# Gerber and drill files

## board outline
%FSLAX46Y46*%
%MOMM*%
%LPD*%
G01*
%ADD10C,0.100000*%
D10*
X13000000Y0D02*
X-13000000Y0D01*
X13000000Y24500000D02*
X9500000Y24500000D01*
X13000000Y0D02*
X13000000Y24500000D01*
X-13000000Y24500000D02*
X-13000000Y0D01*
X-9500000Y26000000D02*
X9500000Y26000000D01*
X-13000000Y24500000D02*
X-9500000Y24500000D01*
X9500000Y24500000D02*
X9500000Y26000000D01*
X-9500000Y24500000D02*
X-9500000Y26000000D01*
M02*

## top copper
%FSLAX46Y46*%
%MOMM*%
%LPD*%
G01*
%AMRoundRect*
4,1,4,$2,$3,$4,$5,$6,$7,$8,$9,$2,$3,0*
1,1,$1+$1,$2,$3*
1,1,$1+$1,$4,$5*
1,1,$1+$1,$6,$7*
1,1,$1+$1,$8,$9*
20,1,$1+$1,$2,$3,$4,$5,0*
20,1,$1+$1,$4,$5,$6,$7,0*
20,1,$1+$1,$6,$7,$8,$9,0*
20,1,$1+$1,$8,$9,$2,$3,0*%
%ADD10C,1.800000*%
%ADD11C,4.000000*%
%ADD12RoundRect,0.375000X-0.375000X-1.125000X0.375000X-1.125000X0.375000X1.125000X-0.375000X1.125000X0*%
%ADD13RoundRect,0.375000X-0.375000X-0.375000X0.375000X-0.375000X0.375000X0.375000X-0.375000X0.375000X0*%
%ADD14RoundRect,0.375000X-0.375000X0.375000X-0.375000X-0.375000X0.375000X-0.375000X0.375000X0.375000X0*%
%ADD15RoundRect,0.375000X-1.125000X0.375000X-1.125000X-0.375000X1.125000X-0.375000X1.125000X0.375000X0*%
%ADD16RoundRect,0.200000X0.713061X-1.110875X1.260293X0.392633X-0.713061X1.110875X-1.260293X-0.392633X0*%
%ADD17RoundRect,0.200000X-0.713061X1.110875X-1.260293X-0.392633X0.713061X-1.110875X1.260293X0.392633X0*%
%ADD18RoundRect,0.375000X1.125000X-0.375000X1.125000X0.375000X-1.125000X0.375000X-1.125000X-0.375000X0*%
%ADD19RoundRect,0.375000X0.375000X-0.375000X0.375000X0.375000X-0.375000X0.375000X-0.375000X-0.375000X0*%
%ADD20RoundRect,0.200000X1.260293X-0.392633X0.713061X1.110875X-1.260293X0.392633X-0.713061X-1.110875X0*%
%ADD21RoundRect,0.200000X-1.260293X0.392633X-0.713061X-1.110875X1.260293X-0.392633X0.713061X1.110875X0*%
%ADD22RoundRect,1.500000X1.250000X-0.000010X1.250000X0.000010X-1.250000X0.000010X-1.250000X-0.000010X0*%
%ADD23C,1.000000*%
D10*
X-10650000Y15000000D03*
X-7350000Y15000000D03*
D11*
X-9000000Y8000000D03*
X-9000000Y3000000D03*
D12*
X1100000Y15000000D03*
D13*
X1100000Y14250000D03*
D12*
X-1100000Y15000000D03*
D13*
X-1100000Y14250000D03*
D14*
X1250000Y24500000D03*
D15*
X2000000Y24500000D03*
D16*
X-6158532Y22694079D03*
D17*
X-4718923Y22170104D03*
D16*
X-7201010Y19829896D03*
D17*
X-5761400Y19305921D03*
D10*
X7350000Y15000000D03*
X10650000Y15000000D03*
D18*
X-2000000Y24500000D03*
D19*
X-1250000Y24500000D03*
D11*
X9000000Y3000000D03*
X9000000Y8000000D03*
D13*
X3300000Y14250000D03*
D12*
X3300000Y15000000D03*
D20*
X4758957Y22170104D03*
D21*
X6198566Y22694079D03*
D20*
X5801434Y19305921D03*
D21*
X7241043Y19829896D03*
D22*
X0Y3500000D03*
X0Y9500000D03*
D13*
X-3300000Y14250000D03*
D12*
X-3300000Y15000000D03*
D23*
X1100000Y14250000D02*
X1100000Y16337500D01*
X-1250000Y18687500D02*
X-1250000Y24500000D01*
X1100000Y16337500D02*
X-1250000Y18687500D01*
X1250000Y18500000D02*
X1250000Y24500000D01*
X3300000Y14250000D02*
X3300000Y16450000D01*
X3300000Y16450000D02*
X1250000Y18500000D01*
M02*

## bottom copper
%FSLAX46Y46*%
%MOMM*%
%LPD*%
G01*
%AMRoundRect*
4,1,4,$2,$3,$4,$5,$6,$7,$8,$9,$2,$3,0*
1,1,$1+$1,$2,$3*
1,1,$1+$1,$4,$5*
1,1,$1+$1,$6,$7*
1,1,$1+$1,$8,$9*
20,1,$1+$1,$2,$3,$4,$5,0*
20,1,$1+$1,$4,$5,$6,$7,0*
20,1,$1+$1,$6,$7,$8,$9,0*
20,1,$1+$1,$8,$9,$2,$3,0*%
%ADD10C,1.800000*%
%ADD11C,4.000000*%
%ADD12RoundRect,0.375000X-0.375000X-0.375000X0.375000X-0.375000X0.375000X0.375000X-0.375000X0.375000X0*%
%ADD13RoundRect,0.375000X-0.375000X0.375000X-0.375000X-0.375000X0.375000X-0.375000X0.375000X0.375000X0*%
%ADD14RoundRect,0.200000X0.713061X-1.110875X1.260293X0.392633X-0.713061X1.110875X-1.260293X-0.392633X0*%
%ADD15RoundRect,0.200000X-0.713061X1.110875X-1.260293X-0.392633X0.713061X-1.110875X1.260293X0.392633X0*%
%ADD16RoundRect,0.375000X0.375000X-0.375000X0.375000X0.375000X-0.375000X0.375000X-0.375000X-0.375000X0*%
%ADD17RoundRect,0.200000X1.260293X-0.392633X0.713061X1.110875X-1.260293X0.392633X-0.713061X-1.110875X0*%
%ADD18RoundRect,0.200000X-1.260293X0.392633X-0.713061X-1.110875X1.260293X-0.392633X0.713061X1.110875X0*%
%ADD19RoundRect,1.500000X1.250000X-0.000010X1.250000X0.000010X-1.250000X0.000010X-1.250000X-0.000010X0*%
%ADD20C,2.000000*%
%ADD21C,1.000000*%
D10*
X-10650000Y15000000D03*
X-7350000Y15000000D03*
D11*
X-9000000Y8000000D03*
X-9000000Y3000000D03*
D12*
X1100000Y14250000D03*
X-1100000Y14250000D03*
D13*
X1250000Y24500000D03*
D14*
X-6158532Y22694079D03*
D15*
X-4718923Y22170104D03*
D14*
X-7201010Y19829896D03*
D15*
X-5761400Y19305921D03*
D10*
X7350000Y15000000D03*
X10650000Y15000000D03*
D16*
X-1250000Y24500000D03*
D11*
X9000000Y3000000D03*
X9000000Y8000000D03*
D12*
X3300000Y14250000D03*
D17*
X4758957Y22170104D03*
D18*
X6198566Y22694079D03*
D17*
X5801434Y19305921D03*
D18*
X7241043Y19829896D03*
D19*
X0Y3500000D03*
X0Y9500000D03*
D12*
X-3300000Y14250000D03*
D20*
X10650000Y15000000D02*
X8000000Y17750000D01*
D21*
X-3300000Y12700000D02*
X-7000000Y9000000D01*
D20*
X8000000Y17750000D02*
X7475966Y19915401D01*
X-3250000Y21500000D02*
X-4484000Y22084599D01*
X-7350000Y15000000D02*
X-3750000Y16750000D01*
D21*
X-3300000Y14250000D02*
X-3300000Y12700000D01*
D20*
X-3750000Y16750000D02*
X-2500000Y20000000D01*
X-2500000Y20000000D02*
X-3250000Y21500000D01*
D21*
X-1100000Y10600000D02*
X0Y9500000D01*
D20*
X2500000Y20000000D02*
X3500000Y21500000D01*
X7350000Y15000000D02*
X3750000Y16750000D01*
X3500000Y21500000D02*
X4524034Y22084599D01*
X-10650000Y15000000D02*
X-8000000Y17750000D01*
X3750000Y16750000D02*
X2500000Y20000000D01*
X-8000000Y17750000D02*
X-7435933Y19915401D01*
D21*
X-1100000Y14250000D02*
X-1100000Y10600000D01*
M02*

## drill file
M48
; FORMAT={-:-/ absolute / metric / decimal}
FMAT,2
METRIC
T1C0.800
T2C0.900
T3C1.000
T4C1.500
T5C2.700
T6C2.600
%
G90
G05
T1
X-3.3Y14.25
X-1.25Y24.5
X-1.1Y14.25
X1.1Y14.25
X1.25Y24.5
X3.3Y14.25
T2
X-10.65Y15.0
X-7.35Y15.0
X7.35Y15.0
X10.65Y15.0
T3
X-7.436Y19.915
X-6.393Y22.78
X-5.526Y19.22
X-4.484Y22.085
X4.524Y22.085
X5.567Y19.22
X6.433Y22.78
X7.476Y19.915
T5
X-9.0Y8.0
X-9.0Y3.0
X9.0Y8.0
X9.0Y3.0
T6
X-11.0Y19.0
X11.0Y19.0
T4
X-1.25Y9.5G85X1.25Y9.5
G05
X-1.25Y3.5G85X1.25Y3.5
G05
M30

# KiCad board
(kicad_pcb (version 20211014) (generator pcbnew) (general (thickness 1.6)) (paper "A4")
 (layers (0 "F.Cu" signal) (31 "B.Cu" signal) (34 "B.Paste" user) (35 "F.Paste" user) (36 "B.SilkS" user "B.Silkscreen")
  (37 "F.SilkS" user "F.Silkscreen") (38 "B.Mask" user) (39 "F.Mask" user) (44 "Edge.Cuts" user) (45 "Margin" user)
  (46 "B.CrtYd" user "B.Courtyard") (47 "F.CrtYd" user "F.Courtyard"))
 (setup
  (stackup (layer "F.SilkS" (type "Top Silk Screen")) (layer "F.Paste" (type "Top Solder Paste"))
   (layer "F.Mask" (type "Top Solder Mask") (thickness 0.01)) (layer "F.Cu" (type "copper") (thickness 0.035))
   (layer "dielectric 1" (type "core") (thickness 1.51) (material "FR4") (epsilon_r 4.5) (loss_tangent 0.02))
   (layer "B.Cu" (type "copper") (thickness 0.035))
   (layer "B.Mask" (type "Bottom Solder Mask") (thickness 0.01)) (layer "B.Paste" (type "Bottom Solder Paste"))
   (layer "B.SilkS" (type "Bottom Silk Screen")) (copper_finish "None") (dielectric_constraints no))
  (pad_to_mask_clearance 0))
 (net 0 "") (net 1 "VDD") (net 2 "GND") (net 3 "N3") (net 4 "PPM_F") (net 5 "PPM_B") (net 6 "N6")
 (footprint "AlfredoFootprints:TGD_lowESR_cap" (layer "F.Cu") (at -9 -15)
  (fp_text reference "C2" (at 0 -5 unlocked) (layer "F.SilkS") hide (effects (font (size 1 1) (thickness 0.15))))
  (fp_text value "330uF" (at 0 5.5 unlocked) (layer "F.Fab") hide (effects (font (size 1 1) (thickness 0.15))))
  (pad "1" thru_hole circle (at -1.65 0) (size 1.8 1.8) (drill 0.9) (layers *.Cu *.Mask) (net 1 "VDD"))
  (pad "2" thru_hole circle (at 1.65 0) (size 1.8 1.8) (drill 0.9) (layers *.Cu *.Mask) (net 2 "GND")))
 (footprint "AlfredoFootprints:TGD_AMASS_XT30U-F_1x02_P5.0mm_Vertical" (layer "F.Cu") (at -9 -5.5 -90)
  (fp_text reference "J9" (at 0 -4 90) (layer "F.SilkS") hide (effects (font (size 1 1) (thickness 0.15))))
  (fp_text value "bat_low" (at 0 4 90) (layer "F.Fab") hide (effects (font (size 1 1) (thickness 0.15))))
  (pad "1" thru_hole circle (at -2.5 0 270) (size 4 4) (drill 2.7) (layers *.Cu *.Mask) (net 2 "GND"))
  (pad "2" thru_hole circle (at 2.5 0 270) (size 4 4) (drill 2.7) (layers *.Cu *.Mask) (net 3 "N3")))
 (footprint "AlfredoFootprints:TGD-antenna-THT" (layer "F.Cu") (at 1.1 -15)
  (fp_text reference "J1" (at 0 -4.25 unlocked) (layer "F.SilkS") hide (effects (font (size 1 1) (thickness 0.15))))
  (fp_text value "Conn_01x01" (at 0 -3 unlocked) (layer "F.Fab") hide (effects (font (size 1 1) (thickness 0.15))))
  (pad "1" smd roundrect (at 0 0) (size 1.5 3) (layers "F.Cu" "F.Paste" "F.Mask") (roundrect_rratio 0.25) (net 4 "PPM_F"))
  (pad "1" thru_hole roundrect (at 0 0.75) (size 1.5 1.5) (drill 0.8) (layers *.Cu *.Mask) (roundrect_rratio 0.25) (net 4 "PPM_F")))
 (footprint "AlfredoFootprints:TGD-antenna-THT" (layer "F.Cu") (at -1.1 -15)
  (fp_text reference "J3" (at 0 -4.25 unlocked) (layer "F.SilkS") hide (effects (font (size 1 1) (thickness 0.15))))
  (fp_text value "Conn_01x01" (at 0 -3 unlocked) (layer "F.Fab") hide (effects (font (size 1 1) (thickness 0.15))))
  (pad "1" smd roundrect (at 0 0) (size 1.5 3) (layers "F.Cu" "F.Paste" "F.Mask") (roundrect_rratio 0.25) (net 1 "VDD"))
  (pad "1" thru_hole roundrect (at 0 0.75) (size 1.5 1.5) (drill 0.8) (layers *.Cu *.Mask) (roundrect_rratio 0.25) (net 1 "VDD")))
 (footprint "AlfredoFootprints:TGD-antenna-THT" (layer "F.Cu") (at 2 -24.5 -90)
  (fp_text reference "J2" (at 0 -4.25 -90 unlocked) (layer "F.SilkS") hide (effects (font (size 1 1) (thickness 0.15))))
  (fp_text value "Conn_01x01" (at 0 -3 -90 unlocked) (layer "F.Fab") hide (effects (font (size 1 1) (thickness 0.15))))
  (pad "1" thru_hole roundrect (at 0 0.75 270) (size 1.5 1.5) (drill 0.8) (layers *.Cu *.Mask) (roundrect_rratio 0.25) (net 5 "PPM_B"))
  (pad "1" smd roundrect (at 0 0 270) (size 1.5 3) (layers "F.Cu" "F.Paste" "F.Mask") (roundrect_rratio 0.25) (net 5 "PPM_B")))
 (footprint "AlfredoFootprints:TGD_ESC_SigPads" (layer "F.Cu") (at -4.484 -22.084599 -110)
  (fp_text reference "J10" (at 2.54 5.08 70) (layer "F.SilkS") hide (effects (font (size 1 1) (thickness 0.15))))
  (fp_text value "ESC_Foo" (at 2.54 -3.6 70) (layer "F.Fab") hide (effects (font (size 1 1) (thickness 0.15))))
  (pad "1" thru_hole roundrect locked (at 0 2.032 70) (size 2 2.5) (drill 1 (offset 0 0.25)) (layers *.Cu *.Mask) (roundrect_rratio 0.1)
   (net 2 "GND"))
  (pad "1" thru_hole roundrect locked (at 0 0 250) (size 2 2.5) (drill 1 (offset 0 0.25)) (layers *.Cu *.Mask) (roundrect_rratio 0.1)
   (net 2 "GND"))
  (pad "2" thru_hole roundrect locked (at 3.048 2.032 70) (size 2 2.5) (drill 1 (offset 0 0.25)) (layers *.Cu *.Mask) (roundrect_rratio 0.1)
   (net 1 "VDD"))
  (pad "2" thru_hole roundrect locked (at 3.048 0 250) (size 2 2.5) (drill 1 (offset 0 0.25)) (layers *.Cu *.Mask) (roundrect_rratio 0.1)
   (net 1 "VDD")))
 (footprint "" (layer "F.Cu") (at 11 -19)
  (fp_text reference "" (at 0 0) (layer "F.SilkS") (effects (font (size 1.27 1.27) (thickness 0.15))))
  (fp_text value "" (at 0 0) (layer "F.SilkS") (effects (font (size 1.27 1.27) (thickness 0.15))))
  (pad "" np_thru_hole circle locked (at 0 0) (size 2.6 2.6) (drill 2.6) (layers F&B.Cu *.Mask)))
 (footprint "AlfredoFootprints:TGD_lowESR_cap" (layer "F.Cu") (at 9 -15)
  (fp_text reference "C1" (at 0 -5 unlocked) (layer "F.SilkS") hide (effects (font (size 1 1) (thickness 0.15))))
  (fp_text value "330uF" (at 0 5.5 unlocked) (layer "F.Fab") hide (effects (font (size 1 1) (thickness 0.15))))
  (pad "1" thru_hole circle (at -1.65 0) (size 1.8 1.8) (drill 0.9) (layers *.Cu *.Mask) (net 1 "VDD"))
  (pad "2" thru_hole circle (at 1.65 0) (size 1.8 1.8) (drill 0.9) (layers *.Cu *.Mask) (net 2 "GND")))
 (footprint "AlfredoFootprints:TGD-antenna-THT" (layer "F.Cu") (at -2 -24.5 90)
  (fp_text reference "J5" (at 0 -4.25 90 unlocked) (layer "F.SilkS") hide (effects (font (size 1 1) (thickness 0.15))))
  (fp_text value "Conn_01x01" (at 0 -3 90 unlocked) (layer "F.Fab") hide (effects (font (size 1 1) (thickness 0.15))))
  (pad "1" smd roundrect (at 0 0 90) (size 1.5 3) (layers "F.Cu" "F.Paste" "F.Mask") (roundrect_rratio 0.25) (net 4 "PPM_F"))
  (pad "1" thru_hole roundrect (at 0 0.75 90) (size 1.5 1.5) (drill 0.8) (layers *.Cu *.Mask) (roundrect_rratio 0.25) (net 4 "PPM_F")))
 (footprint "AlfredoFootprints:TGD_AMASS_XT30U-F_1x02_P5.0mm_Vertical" (layer "F.Cu") (at 9 -5.5 90)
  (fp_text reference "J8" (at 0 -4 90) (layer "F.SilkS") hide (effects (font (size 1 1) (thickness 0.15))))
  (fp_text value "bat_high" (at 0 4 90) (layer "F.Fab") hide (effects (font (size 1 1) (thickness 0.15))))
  (pad "1" thru_hole circle (at -2.5 0 90) (size 4 4) (drill 2.7) (layers *.Cu *.Mask) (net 3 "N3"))
  (pad "2" thru_hole circle (at 2.5 0 90) (size 4 4) (drill 2.7) (layers *.Cu *.Mask) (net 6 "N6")))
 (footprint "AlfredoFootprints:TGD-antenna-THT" (layer "F.Cu") (at 3.3 -15)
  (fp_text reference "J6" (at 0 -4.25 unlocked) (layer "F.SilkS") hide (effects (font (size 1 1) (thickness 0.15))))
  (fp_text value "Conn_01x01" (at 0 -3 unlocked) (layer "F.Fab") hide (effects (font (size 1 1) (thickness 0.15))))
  (pad "1" thru_hole roundrect (at 0 0.75) (size 1.5 1.5) (drill 0.8) (layers *.Cu *.Mask) (roundrect_rratio 0.25) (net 5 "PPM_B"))
  (pad "1" smd roundrect (at 0 0) (size 1.5 3) (layers "F.Cu" "F.Paste" "F.Mask") (roundrect_rratio 0.25) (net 5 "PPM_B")))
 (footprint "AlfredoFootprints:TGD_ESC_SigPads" (layer "F.Cu") (at 6.433489 -22.779584 -70)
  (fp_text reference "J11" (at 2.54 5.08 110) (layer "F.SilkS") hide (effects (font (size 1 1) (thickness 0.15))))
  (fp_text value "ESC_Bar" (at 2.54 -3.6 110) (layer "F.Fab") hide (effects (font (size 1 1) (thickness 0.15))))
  (pad "1" thru_hole roundrect locked (at 0 2.032 110) (size 2 2.5) (drill 1 (offset 0 0.25)) (layers *.Cu *.Mask) (roundrect_rratio 0.1)
   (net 1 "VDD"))
  (pad "1" thru_hole roundrect locked (at 0 0 290) (size 2 2.5) (drill 1 (offset 0 0.25)) (layers *.Cu *.Mask) (roundrect_rratio 0.1)
   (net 1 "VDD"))
  (pad "2" thru_hole roundrect locked (at 3.048 2.032 110) (size 2 2.5) (drill 1 (offset 0 0.25)) (layers *.Cu *.Mask)
   (roundrect_rratio 0.1) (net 2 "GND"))
  (pad "2" thru_hole roundrect locked (at 3.048 0 290) (size 2 2.5) (drill 1 (offset 0 0.25)) (layers *.Cu *.Mask) (roundrect_rratio 0.1)
   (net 2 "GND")))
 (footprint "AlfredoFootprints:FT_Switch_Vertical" (layer "F.Cu") (at 0 -6.5 90)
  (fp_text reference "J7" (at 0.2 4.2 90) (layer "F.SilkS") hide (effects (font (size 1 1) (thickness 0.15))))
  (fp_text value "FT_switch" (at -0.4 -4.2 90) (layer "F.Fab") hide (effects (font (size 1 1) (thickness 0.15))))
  (pad "1" thru_hole roundrect locked (at -3 0 90) (size 3 5.5) (drill oval 1.5 4) (layers *.Cu *.Mask) (roundrect_rratio 0.5) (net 6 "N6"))
  (pad "2" thru_hole roundrect locked (at 3 0 90) (size 3 5.5) (drill oval 1.5 4) (layers *.Cu *.Mask) (roundrect_rratio 0.5) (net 1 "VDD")))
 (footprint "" (layer "F.Cu") (at -11 -19)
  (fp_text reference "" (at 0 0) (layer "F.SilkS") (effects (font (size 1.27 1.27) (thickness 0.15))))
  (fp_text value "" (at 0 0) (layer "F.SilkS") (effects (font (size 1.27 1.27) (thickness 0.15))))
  (pad "" np_thru_hole circle locked (at 0 0) (size 2.6 2.6) (drill 2.6) (layers F&B.Cu *.Mask)))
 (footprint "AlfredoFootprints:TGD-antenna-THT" (layer "F.Cu") (at -3.3 -15)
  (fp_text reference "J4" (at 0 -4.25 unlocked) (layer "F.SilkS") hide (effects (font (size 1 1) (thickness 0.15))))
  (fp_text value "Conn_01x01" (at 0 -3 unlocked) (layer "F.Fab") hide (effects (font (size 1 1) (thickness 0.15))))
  (pad "1" thru_hole roundrect (at 0 0.75) (size 1.5 1.5) (drill 0.8) (layers *.Cu *.Mask) (roundrect_rratio 0.25) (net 2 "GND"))
  (pad "1" smd roundrect (at 0 0) (size 1.5 3) (layers "F.Cu" "F.Paste" "F.Mask") (roundrect_rratio 0.25) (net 2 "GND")))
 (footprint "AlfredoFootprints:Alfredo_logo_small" (layer "B.Cu") (at 0 -19.25 180)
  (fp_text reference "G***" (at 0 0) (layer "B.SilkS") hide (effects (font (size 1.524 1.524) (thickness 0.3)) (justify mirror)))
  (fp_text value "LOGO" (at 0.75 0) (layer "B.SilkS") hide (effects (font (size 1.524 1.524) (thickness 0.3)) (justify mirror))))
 (gr_line (start 13 0) (end -13 0) (layer "Edge.Cuts") (width 0.1))
 (gr_line (start 13 -24.5) (end 9.5 -24.5) (layer "Edge.Cuts") (width 0.1))
 (gr_line (start 13 0) (end 13 -24.5) (layer "Edge.Cuts") (width 0.1))
 (gr_line (start -13 -24.5) (end -13 0) (layer "Edge.Cuts") (width 0.1))
 (gr_line (start -9.5 -26) (end 9.5 -26) (layer "Edge.Cuts") (width 0.1))
 (gr_line (start -13 -24.5) (end -9.5 -24.5) (layer "Edge.Cuts") (width 0.1))
 (gr_line (start 9.5 -24.5) (end 9.5 -26) (layer "Edge.Cuts") (width 0.1))
 (gr_line (start -9.5 -24.5) (end -9.5 -26) (layer "Edge.Cuts") (width 0.1))
 (segment (start 1.1 -14.25) (end 1.1 -16.3375) (width 1) (layer "F.Cu") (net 4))
 (segment (start -1.25 -18.6875) (end -1.25 -24.5) (width 1) (layer "F.Cu") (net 4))
 (segment (start 1.1 -16.3375) (end -1.25 -18.6875) (width 1) (layer "F.Cu") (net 4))
 (segment (start 1.25 -18.5) (end 1.25 -24.5) (width 1) (layer "F.Cu") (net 5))
 (segment (start 3.3 -14.25) (end 3.3 -16.45) (width 1) (layer "F.Cu") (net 5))
 (segment (start 3.3 -16.45) (end 1.25 -18.5) (width 1) (layer "F.Cu") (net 5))
 (segment (start 10.65 -15) (end 8 -17.75) (width 2) (layer "B.Cu") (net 2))
 (segment (start -3.3 -12.7) (end -7 -9) (width 1) (layer "B.Cu") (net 2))
 (segment (start 8 -17.75) (end 7.475966 -19.915401) (width 2) (layer "B.Cu") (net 2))
 (segment (start -3.25 -21.5) (end -4.484 -22.084599) (width 2) (layer "B.Cu") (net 2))
 (segment (start -7.35 -15) (end -3.75 -16.75) (width 2) (layer "B.Cu") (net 2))
 (segment (start -3.3 -14.25) (end -3.3 -12.7) (width 1) (layer "B.Cu") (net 2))
 (segment (start -3.75 -16.75) (end -2.5 -20) (width 2) (layer "B.Cu") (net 2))
 (segment (start -2.5 -20) (end -3.25 -21.5) (width 2) (layer "B.Cu") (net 2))
 (segment (start -1.1 -10.6) (end 0 -9.5) (width 1) (layer "B.Cu") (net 1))
 (segment (start 2.5 -20) (end 3.5 -21.5) (width 2) (layer "B.Cu") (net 1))
 (segment (start 7.35 -15) (end 3.75 -16.75) (width 2) (layer "B.Cu") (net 1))
 (segment (start 3.5 -21.5) (end 4.524034 -22.084599) (width 2) (layer "B.Cu") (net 1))
 (segment (start -10.65 -15) (end -8 -17.75) (width 2) (layer "B.Cu") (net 1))
 (segment (start 3.75 -16.75) (end 2.5 -20) (width 2) (layer "B.Cu") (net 1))
 (segment (start -8 -17.75) (end -7.435933 -19.915401) (width 2) (layer "B.Cu") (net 1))
 (segment (start -1.1 -14.25) (end -1.1 -10.6) (width 1) (layer "B.Cu") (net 1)))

